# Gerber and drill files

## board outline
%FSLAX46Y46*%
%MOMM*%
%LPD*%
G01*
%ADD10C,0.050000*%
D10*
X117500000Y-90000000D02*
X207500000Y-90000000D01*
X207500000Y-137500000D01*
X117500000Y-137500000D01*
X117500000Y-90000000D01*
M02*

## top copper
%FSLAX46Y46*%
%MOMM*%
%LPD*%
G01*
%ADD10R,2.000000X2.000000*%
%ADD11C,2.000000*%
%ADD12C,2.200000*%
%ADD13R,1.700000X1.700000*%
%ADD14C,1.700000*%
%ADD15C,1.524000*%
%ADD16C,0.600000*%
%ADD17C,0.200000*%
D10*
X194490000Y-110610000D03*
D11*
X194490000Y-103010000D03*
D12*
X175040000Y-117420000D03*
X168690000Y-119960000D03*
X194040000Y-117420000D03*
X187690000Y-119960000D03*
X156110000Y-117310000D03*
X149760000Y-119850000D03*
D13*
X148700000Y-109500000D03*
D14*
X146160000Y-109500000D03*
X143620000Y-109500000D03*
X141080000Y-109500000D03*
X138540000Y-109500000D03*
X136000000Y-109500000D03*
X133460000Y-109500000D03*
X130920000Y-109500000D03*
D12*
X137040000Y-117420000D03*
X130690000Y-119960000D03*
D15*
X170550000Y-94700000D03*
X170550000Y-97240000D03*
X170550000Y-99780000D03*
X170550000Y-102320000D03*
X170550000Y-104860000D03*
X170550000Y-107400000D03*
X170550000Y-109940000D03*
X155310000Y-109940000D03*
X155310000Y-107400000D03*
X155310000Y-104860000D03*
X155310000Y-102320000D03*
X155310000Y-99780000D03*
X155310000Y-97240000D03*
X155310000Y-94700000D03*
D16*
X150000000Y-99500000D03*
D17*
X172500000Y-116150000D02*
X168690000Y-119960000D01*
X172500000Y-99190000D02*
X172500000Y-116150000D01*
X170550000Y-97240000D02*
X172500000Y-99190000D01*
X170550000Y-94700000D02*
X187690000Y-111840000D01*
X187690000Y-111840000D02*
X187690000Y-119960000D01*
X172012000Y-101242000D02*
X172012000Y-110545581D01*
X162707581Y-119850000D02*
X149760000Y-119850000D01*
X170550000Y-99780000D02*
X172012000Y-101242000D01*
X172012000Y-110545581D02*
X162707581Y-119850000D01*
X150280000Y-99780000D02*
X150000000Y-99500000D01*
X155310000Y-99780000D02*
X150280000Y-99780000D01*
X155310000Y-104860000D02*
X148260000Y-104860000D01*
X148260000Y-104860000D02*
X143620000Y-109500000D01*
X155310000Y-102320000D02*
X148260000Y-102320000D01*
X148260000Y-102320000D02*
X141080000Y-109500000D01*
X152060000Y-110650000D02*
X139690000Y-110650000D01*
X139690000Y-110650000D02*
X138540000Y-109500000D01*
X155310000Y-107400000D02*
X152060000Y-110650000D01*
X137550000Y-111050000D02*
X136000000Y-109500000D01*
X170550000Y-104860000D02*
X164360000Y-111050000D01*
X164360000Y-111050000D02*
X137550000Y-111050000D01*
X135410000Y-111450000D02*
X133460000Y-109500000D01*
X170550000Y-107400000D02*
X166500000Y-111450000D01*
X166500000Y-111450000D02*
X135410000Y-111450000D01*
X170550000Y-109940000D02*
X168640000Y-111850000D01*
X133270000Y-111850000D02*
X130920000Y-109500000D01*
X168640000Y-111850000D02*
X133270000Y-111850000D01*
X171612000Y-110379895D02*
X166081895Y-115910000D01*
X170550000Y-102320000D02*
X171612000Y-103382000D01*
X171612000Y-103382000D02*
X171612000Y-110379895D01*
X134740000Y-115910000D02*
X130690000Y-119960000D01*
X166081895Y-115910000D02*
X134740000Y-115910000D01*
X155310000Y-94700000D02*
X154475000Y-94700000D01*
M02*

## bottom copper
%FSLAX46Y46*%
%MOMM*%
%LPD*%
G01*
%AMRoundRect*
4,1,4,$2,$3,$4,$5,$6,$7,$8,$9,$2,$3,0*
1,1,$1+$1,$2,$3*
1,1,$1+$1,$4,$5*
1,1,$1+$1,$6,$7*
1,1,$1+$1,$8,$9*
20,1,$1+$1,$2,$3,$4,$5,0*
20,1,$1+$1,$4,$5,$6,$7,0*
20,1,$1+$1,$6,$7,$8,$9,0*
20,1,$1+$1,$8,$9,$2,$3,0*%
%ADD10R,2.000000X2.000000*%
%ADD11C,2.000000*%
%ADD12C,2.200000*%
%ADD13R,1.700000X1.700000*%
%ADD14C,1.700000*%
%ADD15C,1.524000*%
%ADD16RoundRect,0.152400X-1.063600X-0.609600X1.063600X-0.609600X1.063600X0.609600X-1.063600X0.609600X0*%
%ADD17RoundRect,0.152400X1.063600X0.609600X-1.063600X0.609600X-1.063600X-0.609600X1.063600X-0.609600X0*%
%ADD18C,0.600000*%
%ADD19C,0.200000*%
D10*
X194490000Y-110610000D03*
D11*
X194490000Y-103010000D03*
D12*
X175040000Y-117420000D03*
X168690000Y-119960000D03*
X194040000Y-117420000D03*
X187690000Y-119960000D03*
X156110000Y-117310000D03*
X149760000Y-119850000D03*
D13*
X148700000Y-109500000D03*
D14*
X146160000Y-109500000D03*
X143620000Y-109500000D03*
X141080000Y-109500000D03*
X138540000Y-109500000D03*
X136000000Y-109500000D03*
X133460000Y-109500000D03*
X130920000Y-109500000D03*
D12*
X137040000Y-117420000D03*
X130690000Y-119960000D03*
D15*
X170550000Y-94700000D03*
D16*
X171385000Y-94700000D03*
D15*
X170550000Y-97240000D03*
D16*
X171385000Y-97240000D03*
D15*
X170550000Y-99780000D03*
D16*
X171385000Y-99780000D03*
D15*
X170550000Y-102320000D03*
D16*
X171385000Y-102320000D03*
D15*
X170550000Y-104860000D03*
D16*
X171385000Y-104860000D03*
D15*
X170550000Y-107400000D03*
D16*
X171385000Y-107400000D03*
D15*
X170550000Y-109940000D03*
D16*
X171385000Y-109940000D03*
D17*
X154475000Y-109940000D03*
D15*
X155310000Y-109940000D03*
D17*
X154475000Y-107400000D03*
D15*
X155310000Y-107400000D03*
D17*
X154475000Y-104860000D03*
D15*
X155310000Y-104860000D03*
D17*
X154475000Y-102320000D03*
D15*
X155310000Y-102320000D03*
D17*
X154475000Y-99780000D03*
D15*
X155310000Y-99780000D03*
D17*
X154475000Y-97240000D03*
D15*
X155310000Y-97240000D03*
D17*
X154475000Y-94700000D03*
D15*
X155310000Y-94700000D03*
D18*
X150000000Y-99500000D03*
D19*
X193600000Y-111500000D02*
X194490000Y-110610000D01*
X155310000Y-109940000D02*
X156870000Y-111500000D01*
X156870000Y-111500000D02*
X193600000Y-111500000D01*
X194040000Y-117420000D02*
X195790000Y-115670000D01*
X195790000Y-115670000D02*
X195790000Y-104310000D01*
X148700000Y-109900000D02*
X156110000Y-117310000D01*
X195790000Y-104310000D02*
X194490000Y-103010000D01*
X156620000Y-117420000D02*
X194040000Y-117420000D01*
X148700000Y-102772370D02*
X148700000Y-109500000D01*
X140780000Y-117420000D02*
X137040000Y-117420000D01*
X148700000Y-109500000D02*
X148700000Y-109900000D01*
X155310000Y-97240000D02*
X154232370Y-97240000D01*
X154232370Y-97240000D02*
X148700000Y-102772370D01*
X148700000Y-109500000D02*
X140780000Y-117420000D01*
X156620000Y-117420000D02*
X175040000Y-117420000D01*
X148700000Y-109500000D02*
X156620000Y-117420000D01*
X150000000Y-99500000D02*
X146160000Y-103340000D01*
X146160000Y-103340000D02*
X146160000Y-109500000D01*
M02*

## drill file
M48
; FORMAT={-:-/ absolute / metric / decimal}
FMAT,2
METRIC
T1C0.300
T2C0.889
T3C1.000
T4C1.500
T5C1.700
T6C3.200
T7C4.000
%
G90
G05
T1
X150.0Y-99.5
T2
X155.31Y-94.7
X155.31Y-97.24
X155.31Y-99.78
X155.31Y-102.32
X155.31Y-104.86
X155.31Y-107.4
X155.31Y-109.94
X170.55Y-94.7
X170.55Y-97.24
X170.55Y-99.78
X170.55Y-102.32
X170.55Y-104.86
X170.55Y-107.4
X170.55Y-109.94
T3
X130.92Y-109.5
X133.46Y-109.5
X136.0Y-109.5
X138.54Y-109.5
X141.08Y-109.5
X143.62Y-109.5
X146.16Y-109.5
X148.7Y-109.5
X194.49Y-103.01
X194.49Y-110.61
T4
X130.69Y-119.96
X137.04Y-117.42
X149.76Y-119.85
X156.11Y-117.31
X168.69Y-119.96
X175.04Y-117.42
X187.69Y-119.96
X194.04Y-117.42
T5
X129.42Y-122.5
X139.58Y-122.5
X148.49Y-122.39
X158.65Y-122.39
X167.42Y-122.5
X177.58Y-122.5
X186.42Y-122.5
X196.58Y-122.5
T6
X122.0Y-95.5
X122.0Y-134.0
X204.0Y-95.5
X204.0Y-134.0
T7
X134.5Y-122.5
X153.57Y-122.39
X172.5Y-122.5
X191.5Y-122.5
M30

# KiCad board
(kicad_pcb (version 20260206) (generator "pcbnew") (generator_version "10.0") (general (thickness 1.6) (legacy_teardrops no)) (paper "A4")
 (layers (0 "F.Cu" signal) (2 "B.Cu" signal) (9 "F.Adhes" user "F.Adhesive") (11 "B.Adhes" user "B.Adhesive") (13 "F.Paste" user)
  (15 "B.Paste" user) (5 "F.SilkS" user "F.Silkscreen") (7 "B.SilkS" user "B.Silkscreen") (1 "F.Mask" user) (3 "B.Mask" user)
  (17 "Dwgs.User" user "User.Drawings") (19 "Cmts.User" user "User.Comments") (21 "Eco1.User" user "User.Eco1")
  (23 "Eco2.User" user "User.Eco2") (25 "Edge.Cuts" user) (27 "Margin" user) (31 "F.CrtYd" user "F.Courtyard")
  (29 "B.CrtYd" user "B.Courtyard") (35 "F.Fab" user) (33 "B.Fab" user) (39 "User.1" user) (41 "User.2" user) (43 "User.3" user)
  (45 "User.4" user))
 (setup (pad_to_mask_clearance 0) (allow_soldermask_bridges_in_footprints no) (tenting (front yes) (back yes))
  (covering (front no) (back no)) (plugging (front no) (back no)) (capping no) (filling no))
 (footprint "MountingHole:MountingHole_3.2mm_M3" (layer "F.Cu") (at 122 134)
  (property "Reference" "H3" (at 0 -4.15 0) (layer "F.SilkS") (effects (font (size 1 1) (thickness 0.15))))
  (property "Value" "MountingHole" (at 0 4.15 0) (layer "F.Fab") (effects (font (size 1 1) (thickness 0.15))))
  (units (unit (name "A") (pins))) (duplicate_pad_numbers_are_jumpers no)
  (pad "" np_thru_hole circle (at 0 0) (size 3.2 3.2) (drill 3.2) (layers "*.Cu" "*.Mask")))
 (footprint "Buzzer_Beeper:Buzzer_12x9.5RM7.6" (layer "F.Cu") (at 194.49 110.61 90)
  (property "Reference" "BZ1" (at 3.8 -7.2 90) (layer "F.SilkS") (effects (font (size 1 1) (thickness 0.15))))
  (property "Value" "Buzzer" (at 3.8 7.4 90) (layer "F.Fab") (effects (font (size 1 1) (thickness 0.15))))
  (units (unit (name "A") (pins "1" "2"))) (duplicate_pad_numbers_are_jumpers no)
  (pad "1" thru_hole rect (at 0 0 90) (size 2 2) (drill 1) (layers "*.Cu" "*.Mask") (remove_unused_layers no) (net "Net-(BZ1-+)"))
  (pad "2" thru_hole circle (at 7.6 0 90) (size 2 2) (drill 1) (layers "*.Cu" "*.Mask") (remove_unused_layers no) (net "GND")))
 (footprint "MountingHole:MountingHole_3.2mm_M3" (layer "F.Cu") (at 122 95.5)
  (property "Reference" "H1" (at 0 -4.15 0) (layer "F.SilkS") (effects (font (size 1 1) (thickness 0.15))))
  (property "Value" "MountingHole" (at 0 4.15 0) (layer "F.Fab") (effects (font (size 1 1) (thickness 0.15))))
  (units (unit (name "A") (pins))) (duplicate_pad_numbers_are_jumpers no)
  (pad "" np_thru_hole circle (at 0 0) (size 3.2 3.2) (drill 3.2) (layers "*.Cu" "*.Mask")))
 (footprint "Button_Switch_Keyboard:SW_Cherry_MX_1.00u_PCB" (layer "F.Cu") (at 175.04 117.42)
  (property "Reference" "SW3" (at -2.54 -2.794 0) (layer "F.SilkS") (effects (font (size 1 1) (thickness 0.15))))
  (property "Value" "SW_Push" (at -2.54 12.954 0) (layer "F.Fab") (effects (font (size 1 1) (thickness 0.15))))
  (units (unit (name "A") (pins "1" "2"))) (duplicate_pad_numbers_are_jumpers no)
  (pad "" np_thru_hole circle (at -7.62 5.08) (size 1.7 1.7) (drill 1.7) (layers "*.Cu" "*.Mask"))
  (pad "" np_thru_hole circle (at -2.54 5.08) (size 4 4) (drill 4) (layers "*.Cu" "*.Mask"))
  (pad "" np_thru_hole circle (at 2.54 5.08) (size 1.7 1.7) (drill 1.7) (layers "*.Cu" "*.Mask"))
  (pad "1" thru_hole circle (at 0 0) (size 2.2 2.2) (drill 1.5) (layers "*.Cu" "*.Mask") (remove_unused_layers no) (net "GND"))
  (pad "2" thru_hole circle (at -6.35 2.54) (size 2.2 2.2) (drill 1.5) (layers "*.Cu" "*.Mask") (remove_unused_layers no)
   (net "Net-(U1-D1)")))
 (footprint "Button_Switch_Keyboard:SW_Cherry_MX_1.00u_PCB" (layer "F.Cu") (at 194.04 117.42)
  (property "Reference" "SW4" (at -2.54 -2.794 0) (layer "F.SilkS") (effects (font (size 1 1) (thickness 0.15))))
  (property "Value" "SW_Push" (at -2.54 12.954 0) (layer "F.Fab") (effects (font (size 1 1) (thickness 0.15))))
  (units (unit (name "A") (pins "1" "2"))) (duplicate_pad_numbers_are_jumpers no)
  (pad "" np_thru_hole circle (at -7.62 5.08) (size 1.7 1.7) (drill 1.7) (layers "*.Cu" "*.Mask"))
  (pad "" np_thru_hole circle (at -2.54 5.08) (size 4 4) (drill 4) (layers "*.Cu" "*.Mask"))
  (pad "" np_thru_hole circle (at 2.54 5.08) (size 1.7 1.7) (drill 1.7) (layers "*.Cu" "*.Mask"))
  (pad "1" thru_hole circle (at 0 0) (size 2.2 2.2) (drill 1.5) (layers "*.Cu" "*.Mask") (remove_unused_layers no) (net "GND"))
  (pad "2" thru_hole circle (at -6.35 2.54) (size 2.2 2.2) (drill 1.5) (layers "*.Cu" "*.Mask") (remove_unused_layers no)
   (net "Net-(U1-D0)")))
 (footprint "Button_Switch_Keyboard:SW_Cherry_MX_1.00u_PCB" (layer "F.Cu") (at 156.11 117.31)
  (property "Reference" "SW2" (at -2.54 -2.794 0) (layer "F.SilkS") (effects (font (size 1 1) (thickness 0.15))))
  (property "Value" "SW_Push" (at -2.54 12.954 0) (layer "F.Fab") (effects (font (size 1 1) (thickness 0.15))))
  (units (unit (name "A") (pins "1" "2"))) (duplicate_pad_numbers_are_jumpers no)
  (pad "" np_thru_hole circle (at -7.62 5.08) (size 1.7 1.7) (drill 1.7) (layers "*.Cu" "*.Mask"))
  (pad "" np_thru_hole circle (at -2.54 5.08) (size 4 4) (drill 4) (layers "*.Cu" "*.Mask"))
  (pad "" np_thru_hole circle (at 2.54 5.08) (size 1.7 1.7) (drill 1.7) (layers "*.Cu" "*.Mask"))
  (pad "1" thru_hole circle (at 0 0) (size 2.2 2.2) (drill 1.5) (layers "*.Cu" "*.Mask") (remove_unused_layers no) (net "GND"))
  (pad "2" thru_hole circle (at -6.35 2.54) (size 2.2 2.2) (drill 1.5) (layers "*.Cu" "*.Mask") (remove_unused_layers no)
   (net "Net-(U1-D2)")))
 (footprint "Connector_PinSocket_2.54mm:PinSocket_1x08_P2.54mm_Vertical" (layer "F.Cu") (at 148.7 109.5 -90)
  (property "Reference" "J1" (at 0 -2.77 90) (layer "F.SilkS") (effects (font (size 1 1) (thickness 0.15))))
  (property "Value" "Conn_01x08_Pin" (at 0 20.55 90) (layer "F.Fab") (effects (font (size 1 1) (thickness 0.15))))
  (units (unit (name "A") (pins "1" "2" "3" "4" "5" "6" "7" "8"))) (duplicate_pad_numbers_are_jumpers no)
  (pad "1" thru_hole rect (at 0 0 270) (size 1.7 1.7) (drill 1) (layers "*.Cu" "*.Mask") (remove_unused_layers no) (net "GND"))
  (pad "2" thru_hole circle (at 0 2.54 270) (size 1.7 1.7) (drill 1) (layers "*.Cu" "*.Mask") (remove_unused_layers no) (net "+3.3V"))
  (pad "3" thru_hole circle (at 0 5.08 270) (size 1.7 1.7) (drill 1) (layers "*.Cu" "*.Mask") (remove_unused_layers no) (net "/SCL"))
  (pad "4" thru_hole circle (at 0 7.62 270) (size 1.7 1.7) (drill 1) (layers "*.Cu" "*.Mask") (remove_unused_layers no) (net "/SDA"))
  (pad "5" thru_hole circle (at 0 10.16 270) (size 1.7 1.7) (drill 1) (layers "*.Cu" "*.Mask") (remove_unused_layers no) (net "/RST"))
  (pad "6" thru_hole circle (at 0 12.7 270) (size 1.7 1.7) (drill 1) (layers "*.Cu" "*.Mask") (remove_unused_layers no) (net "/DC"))
  (pad "7" thru_hole circle (at 0 15.24 270) (size 1.7 1.7) (drill 1) (layers "*.Cu" "*.Mask") (remove_unused_layers no) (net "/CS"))
  (pad "8" thru_hole circle (at 0 17.78 270) (size 1.7 1.7) (drill 1) (layers "*.Cu" "*.Mask") (remove_unused_layers no) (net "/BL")))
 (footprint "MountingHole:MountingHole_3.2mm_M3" (layer "F.Cu") (at 204 95.5)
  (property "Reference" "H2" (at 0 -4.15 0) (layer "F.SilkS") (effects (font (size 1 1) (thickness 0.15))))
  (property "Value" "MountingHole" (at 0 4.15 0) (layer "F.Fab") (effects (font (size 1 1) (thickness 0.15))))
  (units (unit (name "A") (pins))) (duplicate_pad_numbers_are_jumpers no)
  (pad "" np_thru_hole circle (at 0 0) (size 3.2 3.2) (drill 3.2) (layers "*.Cu" "*.Mask")))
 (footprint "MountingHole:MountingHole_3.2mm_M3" (layer "F.Cu") (at 204 134)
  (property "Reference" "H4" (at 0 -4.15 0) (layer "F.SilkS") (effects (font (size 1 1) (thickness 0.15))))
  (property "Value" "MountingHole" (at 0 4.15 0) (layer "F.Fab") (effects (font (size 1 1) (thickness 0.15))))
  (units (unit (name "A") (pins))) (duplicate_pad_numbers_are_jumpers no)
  (pad "" np_thru_hole circle (at 0 0) (size 3.2 3.2) (drill 3.2) (layers "*.Cu" "*.Mask")))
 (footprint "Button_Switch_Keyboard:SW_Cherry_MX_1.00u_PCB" (layer "F.Cu") (at 137.04 117.42)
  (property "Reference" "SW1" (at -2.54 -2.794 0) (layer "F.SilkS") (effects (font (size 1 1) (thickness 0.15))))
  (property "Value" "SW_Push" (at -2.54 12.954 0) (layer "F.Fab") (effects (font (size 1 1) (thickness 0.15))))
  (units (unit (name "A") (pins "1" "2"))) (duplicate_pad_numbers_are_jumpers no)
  (pad "" np_thru_hole circle (at -7.62 5.08) (size 1.7 1.7) (drill 1.7) (layers "*.Cu" "*.Mask"))
  (pad "" np_thru_hole circle (at -2.54 5.08) (size 4 4) (drill 4) (layers "*.Cu" "*.Mask"))
  (pad "" np_thru_hole circle (at 2.54 5.08) (size 1.7 1.7) (drill 1.7) (layers "*.Cu" "*.Mask"))
  (pad "1" thru_hole circle (at 0 0) (size 2.2 2.2) (drill 1.5) (layers "*.Cu" "*.Mask") (remove_unused_layers no) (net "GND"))
  (pad "2" thru_hole circle (at -6.35 2.54) (size 2.2 2.2) (drill 1.5) (layers "*.Cu" "*.Mask") (remove_unused_layers no)
   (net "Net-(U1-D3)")))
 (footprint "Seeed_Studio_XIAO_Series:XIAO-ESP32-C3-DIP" (layer "B.Cu") (at 162.93 102.32 90)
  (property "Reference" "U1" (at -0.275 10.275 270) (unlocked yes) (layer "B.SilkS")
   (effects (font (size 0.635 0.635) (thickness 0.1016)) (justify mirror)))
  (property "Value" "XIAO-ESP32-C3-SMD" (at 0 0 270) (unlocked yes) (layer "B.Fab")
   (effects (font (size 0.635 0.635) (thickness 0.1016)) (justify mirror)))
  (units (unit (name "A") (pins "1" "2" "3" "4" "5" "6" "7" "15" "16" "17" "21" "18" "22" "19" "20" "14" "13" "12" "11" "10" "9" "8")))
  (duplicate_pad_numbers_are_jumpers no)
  (pad "1" thru_hole circle (at 7.62 7.62) (size 1.524 1.524) (drill 0.889) (layers "*.Cu" "*.Mask") (remove_unused_layers no)
   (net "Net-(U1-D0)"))
  (pad "1" smd roundrect (at 7.62 8.455) (size 2.432 1.524) (layers "B.Cu" "B.Mask") (roundrect_rratio 0.1) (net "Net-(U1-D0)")
   (thermal_bridge_angle 45))
  (pad "2" thru_hole circle (at 5.08 7.62) (size 1.524 1.524) (drill 0.889) (layers "*.Cu" "*.Mask") (remove_unused_layers no)
   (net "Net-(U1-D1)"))
  (pad "2" smd roundrect (at 5.08 8.455) (size 2.432 1.524) (layers "B.Cu" "B.Mask") (roundrect_rratio 0.1) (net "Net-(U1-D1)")
   (thermal_bridge_angle 45))
  (pad "3" thru_hole circle (at 2.54 7.62) (size 1.524 1.524) (drill 0.889) (layers "*.Cu" "*.Mask") (remove_unused_layers no)
   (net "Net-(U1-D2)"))
  (pad "3" smd roundrect (at 2.54 8.455) (size 2.432 1.524) (layers "B.Cu" "B.Mask") (roundrect_rratio 0.1) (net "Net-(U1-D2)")
   (thermal_bridge_angle 45))
  (pad "4" thru_hole circle (at 0 7.62) (size 1.524 1.524) (drill 0.889) (layers "*.Cu" "*.Mask") (remove_unused_layers no)
   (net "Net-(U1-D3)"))
  (pad "4" smd roundrect (at 0 8.455) (size 2.432 1.524) (layers "B.Cu" "B.Mask") (roundrect_rratio 0.1) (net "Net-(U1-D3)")
   (thermal_bridge_angle 45))
  (pad "5" thru_hole circle (at -2.54 7.62) (size 1.524 1.524) (drill 0.889) (layers "*.Cu" "*.Mask") (remove_unused_layers no) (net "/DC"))
  (pad "5" smd roundrect (at -2.54 8.455) (size 2.432 1.524) (layers "B.Cu" "B.Mask") (roundrect_rratio 0.1) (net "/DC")
   (thermal_bridge_angle 45))
  (pad "6" thru_hole circle (at -5.08 7.62) (size 1.524 1.524) (drill 0.889) (layers "*.Cu" "*.Mask") (remove_unused_layers no) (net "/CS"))
  (pad "6" smd roundrect (at -5.08 8.455) (size 2.432 1.524) (layers "B.Cu" "B.Mask") (roundrect_rratio 0.1) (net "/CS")
   (thermal_bridge_angle 45))
  (pad "7" thru_hole circle (at -7.62 7.62) (size 1.524 1.524) (drill 0.889) (layers "*.Cu" "*.Mask") (remove_unused_layers no) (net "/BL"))
  (pad "7" smd roundrect (at -7.62 8.455) (size 2.432 1.524) (layers "B.Cu" "B.Mask") (roundrect_rratio 0.1) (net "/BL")
   (thermal_bridge_angle 45))
  (pad "8" smd roundrect (at -7.62 -8.455 180) (size 2.432 1.524) (layers "B.Cu" "B.Mask") (roundrect_rratio 0.1) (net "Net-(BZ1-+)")
   (thermal_bridge_angle 45))
  (pad "8" thru_hole circle (at -7.62 -7.62 180) (size 1.524 1.524) (drill 0.889) (layers "*.Cu" "*.Mask") (remove_unused_layers no)
   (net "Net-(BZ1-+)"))
  (pad "9" smd roundrect (at -5.08 -8.455 180) (size 2.432 1.524) (layers "B.Cu" "B.Mask") (roundrect_rratio 0.1) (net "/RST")
   (thermal_bridge_angle 45))
  (pad "9" thru_hole circle (at -5.08 -7.62 180) (size 1.524 1.524) (drill 0.889) (layers "*.Cu" "*.Mask") (remove_unused_layers no)
   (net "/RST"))
  (pad "10" smd roundrect (at -2.54 -8.455 180) (size 2.432 1.524) (layers "B.Cu" "B.Mask") (roundrect_rratio 0.1) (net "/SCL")
   (thermal_bridge_angle 45))
  (pad "10" thru_hole circle (at -2.54 -7.62 180) (size 1.524 1.524) (drill 0.889) (layers "*.Cu" "*.Mask") (remove_unused_layers no)
   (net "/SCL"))
  (pad "11" smd roundrect (at 0 -8.455 180) (size 2.432 1.524) (layers "B.Cu" "B.Mask") (roundrect_rratio 0.1) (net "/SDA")
   (thermal_bridge_angle 45))
  (pad "11" thru_hole circle (at 0 -7.62 180) (size 1.524 1.524) (drill 0.889) (layers "*.Cu" "*.Mask") (remove_unused_layers no)
   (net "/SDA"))
  (pad "12" smd roundrect (at 2.54 -8.455 180) (size 2.432 1.524) (layers "B.Cu" "B.Mask") (roundrect_rratio 0.1) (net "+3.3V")
   (thermal_bridge_angle 45))
  (pad "12" thru_hole circle (at 2.54 -7.62 180) (size 1.524 1.524) (drill 0.889) (layers "*.Cu" "*.Mask") (remove_unused_layers no)
   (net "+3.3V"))
  (pad "13" smd roundrect (at 5.08 -8.455 180) (size 2.432 1.524) (layers "B.Cu" "B.Mask") (roundrect_rratio 0.1) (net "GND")
   (thermal_bridge_angle 45))
  (pad "13" thru_hole circle (at 5.08 -7.62 180) (size 1.524 1.524) (drill 0.889) (layers "*.Cu" "*.Mask") (remove_unused_layers no)
   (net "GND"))
  (pad "14" smd roundrect (at 7.62 -8.455 180) (size 2.432 1.524) (layers "B.Cu" "B.Mask") (roundrect_rratio 0.1)
   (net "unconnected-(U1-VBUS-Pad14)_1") (thermal_bridge_angle 45))
  (pad "14" thru_hole circle (at 7.62 -7.62 180) (size 1.524 1.524) (drill 0.889) (layers "*.Cu" "*.Mask") (remove_unused_layers no)
   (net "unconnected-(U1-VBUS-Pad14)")))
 (gr_rect (start 117.5 90) (end 207.5 137.5) (stroke (width 0.05) (type default)) (fill no) (layer "Edge.Cuts"))
 (segment (start 193.6 111.5) (end 194.49 110.61) (width 0.2) (layer "B.Cu") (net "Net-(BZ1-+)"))
 (segment (start 155.31 109.94) (end 156.87 111.5) (width 0.2) (layer "B.Cu") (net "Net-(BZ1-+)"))
 (segment (start 156.87 111.5) (end 193.6 111.5) (width 0.2) (layer "B.Cu") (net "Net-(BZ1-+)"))
 (segment (start 194.04 117.42) (end 195.79 115.67) (width 0.2) (layer "B.Cu") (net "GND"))
 (segment (start 195.79 115.67) (end 195.79 104.31) (width 0.2) (layer "B.Cu") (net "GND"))
 (segment (start 148.7 109.9) (end 156.11 117.31) (width 0.2) (layer "B.Cu") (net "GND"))
 (segment (start 195.79 104.31) (end 194.49 103.01) (width 0.2) (layer "B.Cu") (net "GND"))
 (segment (start 156.62 117.42) (end 194.04 117.42) (width 0.2) (layer "B.Cu") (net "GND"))
 (segment (start 148.7 102.77237) (end 148.7 109.5) (width 0.2) (layer "B.Cu") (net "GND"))
 (segment (start 140.78 117.42) (end 137.04 117.42) (width 0.2) (layer "B.Cu") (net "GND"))
 (segment (start 148.7 109.5) (end 148.7 109.9) (width 0.2) (layer "B.Cu") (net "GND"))
 (segment (start 155.31 97.24) (end 154.23237 97.24) (width 0.2) (layer "B.Cu") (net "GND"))
 (segment (start 154.23237 97.24) (end 148.7 102.77237) (width 0.2) (layer "B.Cu") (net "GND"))
 (segment (start 148.7 109.5) (end 140.78 117.42) (width 0.2) (layer "B.Cu") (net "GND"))
 (segment (start 156.62 117.42) (end 175.04 117.42) (width 0.2) (layer "B.Cu") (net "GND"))
 (segment (start 148.7 109.5) (end 156.62 117.42) (width 0.2) (layer "B.Cu") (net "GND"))
 (segment (start 172.5 116.15) (end 168.69 119.96) (width 0.2) (layer "F.Cu") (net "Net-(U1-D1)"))
 (segment (start 172.5 99.19) (end 172.5 116.15) (width 0.2) (layer "F.Cu") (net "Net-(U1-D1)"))
 (segment (start 170.55 97.24) (end 172.5 99.19) (width 0.2) (layer "F.Cu") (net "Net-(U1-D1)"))
 (segment (start 170.55 94.7) (end 187.69 111.84) (width 0.2) (layer "F.Cu") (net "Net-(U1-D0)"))
 (segment (start 187.69 111.84) (end 187.69 119.96) (width 0.2) (layer "F.Cu") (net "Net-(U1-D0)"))
 (segment (start 172.012 101.242) (end 172.012 110.545581) (width 0.2) (layer "F.Cu") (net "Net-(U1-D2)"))
 (segment (start 162.707581 119.85) (end 149.76 119.85) (width 0.2) (layer "F.Cu") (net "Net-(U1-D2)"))
 (segment (start 170.55 99.78) (end 172.012 101.242) (width 0.2) (layer "F.Cu") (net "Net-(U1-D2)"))
 (segment (start 172.012 110.545581) (end 162.707581 119.85) (width 0.2) (layer "F.Cu") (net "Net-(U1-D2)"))
 (segment (start 150.28 99.78) (end 150 99.5) (width 0.2) (layer "F.Cu") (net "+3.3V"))
 (segment (start 155.31 99.78) (end 150.28 99.78) (width 0.2) (layer "F.Cu") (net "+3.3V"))
 (via (at 150 99.5) (size 0.6) (drill 0.3) (layers "F.Cu" "B.Cu") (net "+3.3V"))
 (segment (start 150 99.5) (end 146.16 103.34) (width 0.2) (layer "B.Cu") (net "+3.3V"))
 (segment (start 146.16 103.34) (end 146.16 109.5) (width 0.2) (layer "B.Cu") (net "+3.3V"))
 (segment (start 155.31 104.86) (end 148.26 104.86) (width 0.2) (layer "F.Cu") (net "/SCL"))
 (segment (start 148.26 104.86) (end 143.62 109.5) (width 0.2) (layer "F.Cu") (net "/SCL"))
 (segment (start 155.31 102.32) (end 148.26 102.32) (width 0.2) (layer "F.Cu") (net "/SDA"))
 (segment (start 148.26 102.32) (end 141.08 109.5) (width 0.2) (layer "F.Cu") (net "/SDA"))
 (segment (start 152.06 110.65) (end 139.69 110.65) (width 0.2) (layer "F.Cu") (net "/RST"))
 (segment (start 139.69 110.65) (end 138.54 109.5) (width 0.2) (layer "F.Cu") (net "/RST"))
 (segment (start 155.31 107.4) (end 152.06 110.65) (width 0.2) (layer "F.Cu") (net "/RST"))
 (segment (start 137.55 111.05) (end 136 109.5) (width 0.2) (layer "F.Cu") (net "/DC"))
 (segment (start 170.55 104.86) (end 164.36 111.05) (width 0.2) (layer "F.Cu") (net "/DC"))
 (segment (start 164.36 111.05) (end 137.55 111.05) (width 0.2) (layer "F.Cu") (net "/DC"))
 (segment (start 135.41 111.45) (end 133.46 109.5) (width 0.2) (layer "F.Cu") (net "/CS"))
 (segment (start 170.55 107.4) (end 166.5 111.45) (width 0.2) (layer "F.Cu") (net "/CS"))
 (segment (start 166.5 111.45) (end 135.41 111.45) (width 0.2) (layer "F.Cu") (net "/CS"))
 (segment (start 170.55 109.94) (end 168.64 111.85) (width 0.2) (layer "F.Cu") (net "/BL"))
 (segment (start 133.27 111.85) (end 130.92 109.5) (width 0.2) (layer "F.Cu") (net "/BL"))
 (segment (start 168.64 111.85) (end 133.27 111.85) (width 0.2) (layer "F.Cu") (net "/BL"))
 (segment (start 171.612 110.379895) (end 166.081895 115.91) (width 0.2) (layer "F.Cu") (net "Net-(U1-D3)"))
 (segment (start 170.55 102.32) (end 171.612 103.382) (width 0.2) (layer "F.Cu") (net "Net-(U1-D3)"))
 (segment (start 171.612 103.382) (end 171.612 110.379895) (width 0.2) (layer "F.Cu") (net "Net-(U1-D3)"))
 (segment (start 134.74 115.91) (end 130.69 119.96) (width 0.2) (layer "F.Cu") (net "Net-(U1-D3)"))
 (segment (start 166.081895 115.91) (end 134.74 115.91) (width 0.2) (layer "F.Cu") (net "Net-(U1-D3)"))
 (segment (start 155.31 94.7) (end 154.475 94.7) (width 0.2) (layer "F.Cu") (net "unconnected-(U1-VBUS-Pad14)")))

